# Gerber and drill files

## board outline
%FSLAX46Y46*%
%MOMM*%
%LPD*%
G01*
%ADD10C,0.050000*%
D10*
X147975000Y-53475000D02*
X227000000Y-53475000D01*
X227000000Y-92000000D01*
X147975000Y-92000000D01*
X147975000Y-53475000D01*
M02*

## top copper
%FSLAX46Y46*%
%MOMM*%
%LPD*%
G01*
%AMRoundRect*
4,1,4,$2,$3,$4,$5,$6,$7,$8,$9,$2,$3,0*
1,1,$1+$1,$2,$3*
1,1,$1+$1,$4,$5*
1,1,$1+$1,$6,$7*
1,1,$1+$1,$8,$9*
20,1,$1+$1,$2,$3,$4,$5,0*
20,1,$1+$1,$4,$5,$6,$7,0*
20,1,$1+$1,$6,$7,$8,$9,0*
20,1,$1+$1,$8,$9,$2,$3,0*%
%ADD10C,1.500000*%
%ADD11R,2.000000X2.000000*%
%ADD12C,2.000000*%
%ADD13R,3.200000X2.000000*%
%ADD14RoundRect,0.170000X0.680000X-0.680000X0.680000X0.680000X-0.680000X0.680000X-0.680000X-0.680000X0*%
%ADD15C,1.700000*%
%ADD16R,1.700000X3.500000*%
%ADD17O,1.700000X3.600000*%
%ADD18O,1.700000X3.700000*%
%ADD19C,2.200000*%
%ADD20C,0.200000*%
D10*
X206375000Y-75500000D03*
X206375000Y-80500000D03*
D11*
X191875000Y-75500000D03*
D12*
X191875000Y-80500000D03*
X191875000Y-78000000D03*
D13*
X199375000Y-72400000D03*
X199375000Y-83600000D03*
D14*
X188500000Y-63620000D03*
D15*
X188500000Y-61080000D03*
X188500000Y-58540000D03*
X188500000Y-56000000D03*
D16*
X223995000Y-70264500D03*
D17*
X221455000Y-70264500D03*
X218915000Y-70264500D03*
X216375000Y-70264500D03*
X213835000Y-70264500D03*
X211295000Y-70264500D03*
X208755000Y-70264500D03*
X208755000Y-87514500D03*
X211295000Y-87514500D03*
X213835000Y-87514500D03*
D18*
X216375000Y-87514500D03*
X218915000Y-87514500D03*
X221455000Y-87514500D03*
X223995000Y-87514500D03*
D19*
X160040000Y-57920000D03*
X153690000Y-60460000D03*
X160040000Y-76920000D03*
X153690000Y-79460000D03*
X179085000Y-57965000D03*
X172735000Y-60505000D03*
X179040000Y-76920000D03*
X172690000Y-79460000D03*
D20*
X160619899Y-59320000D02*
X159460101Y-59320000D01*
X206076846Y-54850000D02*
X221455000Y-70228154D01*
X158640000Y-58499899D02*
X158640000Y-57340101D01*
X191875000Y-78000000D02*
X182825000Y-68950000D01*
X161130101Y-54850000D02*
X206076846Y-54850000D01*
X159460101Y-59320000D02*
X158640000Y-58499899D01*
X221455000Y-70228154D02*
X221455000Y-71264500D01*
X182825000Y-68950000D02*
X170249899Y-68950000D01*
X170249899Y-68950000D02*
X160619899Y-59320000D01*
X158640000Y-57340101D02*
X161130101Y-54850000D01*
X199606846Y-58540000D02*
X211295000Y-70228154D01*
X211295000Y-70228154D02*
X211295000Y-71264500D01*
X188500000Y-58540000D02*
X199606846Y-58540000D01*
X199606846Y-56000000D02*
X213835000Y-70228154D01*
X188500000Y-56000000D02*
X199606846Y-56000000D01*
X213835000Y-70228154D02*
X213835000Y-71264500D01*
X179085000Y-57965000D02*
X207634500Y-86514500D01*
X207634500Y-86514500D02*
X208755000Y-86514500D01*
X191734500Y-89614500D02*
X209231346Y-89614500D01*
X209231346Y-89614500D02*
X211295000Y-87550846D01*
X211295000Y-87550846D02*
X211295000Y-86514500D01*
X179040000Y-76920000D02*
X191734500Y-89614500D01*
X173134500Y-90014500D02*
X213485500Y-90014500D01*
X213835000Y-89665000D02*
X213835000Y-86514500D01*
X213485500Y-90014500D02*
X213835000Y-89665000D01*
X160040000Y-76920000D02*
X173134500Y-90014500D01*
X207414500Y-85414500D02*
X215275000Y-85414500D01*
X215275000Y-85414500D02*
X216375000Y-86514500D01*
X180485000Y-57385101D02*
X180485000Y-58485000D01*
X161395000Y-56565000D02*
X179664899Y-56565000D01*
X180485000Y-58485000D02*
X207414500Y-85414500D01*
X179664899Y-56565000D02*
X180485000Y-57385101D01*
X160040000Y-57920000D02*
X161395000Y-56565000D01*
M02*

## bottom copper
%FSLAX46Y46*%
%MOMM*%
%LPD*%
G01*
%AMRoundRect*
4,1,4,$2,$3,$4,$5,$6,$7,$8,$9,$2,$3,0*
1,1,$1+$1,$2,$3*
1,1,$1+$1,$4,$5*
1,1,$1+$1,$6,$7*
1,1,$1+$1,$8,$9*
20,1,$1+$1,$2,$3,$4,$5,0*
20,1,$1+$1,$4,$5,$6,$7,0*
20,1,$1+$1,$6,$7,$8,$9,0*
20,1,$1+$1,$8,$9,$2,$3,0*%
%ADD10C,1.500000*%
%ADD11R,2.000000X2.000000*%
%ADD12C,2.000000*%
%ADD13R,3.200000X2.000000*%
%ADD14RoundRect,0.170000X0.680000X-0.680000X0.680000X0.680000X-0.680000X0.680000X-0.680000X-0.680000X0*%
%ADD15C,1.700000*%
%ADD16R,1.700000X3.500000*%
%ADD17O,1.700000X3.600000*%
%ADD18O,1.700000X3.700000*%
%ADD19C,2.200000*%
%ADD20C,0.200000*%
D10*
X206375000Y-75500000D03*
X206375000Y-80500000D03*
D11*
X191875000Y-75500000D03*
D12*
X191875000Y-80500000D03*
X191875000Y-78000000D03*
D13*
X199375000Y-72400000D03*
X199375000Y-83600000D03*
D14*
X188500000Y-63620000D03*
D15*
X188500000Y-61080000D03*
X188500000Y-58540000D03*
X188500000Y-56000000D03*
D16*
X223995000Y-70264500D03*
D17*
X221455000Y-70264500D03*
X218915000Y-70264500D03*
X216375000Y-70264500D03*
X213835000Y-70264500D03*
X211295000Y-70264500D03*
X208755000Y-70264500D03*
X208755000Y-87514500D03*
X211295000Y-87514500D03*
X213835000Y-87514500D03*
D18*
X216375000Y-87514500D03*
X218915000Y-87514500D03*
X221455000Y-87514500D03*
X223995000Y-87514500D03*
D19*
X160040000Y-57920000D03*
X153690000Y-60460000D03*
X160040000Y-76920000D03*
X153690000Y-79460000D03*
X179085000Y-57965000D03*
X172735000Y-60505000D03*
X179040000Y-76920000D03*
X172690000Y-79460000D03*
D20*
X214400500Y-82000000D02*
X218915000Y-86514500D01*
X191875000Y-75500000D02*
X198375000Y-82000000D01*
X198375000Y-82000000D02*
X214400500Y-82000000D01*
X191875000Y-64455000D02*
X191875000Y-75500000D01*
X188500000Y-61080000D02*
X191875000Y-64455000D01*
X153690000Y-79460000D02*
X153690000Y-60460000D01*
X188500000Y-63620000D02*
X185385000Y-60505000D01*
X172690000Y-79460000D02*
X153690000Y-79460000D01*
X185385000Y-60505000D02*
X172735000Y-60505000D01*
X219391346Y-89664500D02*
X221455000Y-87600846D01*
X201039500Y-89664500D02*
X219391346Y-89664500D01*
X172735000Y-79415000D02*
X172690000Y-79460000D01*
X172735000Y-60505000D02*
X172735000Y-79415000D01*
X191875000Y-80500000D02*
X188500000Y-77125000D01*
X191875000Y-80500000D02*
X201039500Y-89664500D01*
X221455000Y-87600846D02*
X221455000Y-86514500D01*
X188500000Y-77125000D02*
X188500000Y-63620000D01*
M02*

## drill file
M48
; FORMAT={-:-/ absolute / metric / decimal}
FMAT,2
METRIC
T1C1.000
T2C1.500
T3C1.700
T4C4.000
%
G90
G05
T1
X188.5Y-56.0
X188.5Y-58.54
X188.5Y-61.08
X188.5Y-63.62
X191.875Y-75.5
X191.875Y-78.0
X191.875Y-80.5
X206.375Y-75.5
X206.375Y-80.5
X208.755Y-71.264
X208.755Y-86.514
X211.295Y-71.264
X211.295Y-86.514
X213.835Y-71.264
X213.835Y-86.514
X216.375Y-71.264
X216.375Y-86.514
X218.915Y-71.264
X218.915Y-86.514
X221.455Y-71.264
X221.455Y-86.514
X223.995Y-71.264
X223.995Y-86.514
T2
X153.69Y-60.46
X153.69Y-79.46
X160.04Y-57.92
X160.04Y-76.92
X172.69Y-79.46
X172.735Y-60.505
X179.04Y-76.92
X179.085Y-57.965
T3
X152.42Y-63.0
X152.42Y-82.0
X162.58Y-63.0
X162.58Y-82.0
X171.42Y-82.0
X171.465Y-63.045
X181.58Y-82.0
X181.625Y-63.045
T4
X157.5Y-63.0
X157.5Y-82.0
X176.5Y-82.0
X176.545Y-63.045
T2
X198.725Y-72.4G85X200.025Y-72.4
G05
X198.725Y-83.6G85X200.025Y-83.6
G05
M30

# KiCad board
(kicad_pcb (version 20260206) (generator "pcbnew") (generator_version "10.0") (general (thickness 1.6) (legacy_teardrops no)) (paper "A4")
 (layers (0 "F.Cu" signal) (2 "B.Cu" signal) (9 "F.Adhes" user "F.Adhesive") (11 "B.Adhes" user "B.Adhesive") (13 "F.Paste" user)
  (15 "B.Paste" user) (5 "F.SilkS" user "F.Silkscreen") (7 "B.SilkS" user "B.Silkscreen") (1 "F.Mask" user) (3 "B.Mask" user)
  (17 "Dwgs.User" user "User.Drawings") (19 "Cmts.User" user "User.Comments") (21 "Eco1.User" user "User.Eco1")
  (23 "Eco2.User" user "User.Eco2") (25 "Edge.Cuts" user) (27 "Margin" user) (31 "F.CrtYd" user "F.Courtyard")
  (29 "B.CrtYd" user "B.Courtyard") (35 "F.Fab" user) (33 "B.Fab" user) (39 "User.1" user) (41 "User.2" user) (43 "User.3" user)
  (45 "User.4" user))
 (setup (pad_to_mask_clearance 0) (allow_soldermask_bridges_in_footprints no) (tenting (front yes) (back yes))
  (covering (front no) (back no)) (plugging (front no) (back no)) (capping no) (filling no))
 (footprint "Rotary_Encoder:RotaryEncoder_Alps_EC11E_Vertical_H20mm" (layer "F.Cu") (at 191.875 75.5)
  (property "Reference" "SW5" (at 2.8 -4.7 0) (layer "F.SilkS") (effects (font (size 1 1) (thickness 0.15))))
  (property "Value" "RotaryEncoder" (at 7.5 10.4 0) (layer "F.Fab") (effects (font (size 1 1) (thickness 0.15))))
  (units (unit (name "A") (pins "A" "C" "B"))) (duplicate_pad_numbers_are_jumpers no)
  (pad "" thru_hole circle (at 14.5 0) (size 1.5 1.5) (drill 1) (layers "*.Cu" "*.Mask") (remove_unused_layers no))
  (pad "" thru_hole circle (at 14.5 5) (size 1.5 1.5) (drill 1) (layers "*.Cu" "*.Mask") (remove_unused_layers no))
  (pad "A" thru_hole rect (at 0 0) (size 2 2) (drill 1) (layers "*.Cu" "*.Mask") (remove_unused_layers no) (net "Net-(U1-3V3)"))
  (pad "B" thru_hole circle (at 0 5) (size 2 2) (drill 1) (layers "*.Cu" "*.Mask") (remove_unused_layers no) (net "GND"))
  (pad "C" thru_hole circle (at 0 2.5) (size 2 2) (drill 1) (layers "*.Cu" "*.Mask") (remove_unused_layers no) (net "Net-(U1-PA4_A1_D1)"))
  (pad "MP" thru_hole rect (at 7.5 -3.1) (size 3.2 2) (drill oval 2.8 1.5) (layers "*.Cu" "*.Mask") (remove_unused_layers no))
  (pad "MP" thru_hole rect (at 7.5 8.1) (size 3.2 2) (drill oval 2.8 1.5) (layers "*.Cu" "*.Mask") (remove_unused_layers no)))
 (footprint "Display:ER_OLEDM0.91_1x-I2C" (layer "F.Cu") (at 188.5 63.62 90)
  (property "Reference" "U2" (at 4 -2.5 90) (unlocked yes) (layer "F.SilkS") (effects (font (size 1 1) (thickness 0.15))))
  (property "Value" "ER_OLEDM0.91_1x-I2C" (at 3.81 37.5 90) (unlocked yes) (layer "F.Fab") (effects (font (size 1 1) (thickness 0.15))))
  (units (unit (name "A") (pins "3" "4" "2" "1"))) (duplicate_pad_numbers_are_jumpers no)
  (pad "1" thru_hole roundrect (at 0 0 90) (size 1.7 1.7) (drill 1) (layers "*.Cu" "*.Mask") (remove_unused_layers no)
   (roundrect_rratio 0.1) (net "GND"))
  (pad "2" thru_hole circle (at 2.54 0 90) (size 1.7 1.7) (drill 1) (layers "*.Cu" "*.Mask") (remove_unused_layers no) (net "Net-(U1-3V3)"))
  (pad "3" thru_hole circle (at 5.08 0 90) (size 1.7 1.7) (drill 1) (layers "*.Cu" "*.Mask") (remove_unused_layers no)
   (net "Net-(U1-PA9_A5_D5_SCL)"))
  (pad "4" thru_hole circle (at 7.62 0 90) (size 1.7 1.7) (drill 1) (layers "*.Cu" "*.Mask") (remove_unused_layers no)
   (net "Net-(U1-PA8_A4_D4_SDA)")))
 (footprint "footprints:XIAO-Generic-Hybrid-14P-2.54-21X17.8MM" (layer "F.Cu") (at 216.375 78.8895 -90)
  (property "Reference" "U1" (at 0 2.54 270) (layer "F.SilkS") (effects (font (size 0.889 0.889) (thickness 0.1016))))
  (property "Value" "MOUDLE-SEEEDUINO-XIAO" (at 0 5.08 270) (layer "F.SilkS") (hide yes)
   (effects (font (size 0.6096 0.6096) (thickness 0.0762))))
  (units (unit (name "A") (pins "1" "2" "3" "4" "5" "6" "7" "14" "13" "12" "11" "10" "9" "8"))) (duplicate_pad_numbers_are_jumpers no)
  (pad "1" thru_hole rect (at -7.625 -7.62 270) (size 3.5 1.7) (drill 1 (offset -1 0)) (layers "*.Cu" "*.Mask") (remove_unused_layers no)
   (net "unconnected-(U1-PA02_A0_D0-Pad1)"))
  (pad "2" thru_hole oval (at -7.625 -5.08 270) (size 3.6 1.7) (drill 1 (offset -1 0)) (layers "*.Cu" "*.Mask") (remove_unused_layers no)
   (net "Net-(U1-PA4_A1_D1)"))
  (pad "3" thru_hole oval (at -7.625 -2.54 270) (size 3.6 1.7) (drill 1 (offset -1 0)) (layers "*.Cu" "*.Mask") (remove_unused_layers no)
   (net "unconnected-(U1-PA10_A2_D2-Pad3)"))
  (pad "4" thru_hole oval (at -7.625 0 270) (size 3.6 1.7) (drill 1 (offset -1 0)) (layers "*.Cu" "*.Mask") (remove_unused_layers no)
   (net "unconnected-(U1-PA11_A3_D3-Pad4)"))
  (pad "5" thru_hole oval (at -7.625 2.54 270) (size 3.6 1.7) (drill 1 (offset -1 0)) (layers "*.Cu" "*.Mask") (remove_unused_layers no)
   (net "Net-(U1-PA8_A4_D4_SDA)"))
  (pad "6" thru_hole oval (at -7.625 5.08 90) (size 3.6 1.7) (drill 1 (offset 1 0)) (layers "*.Cu" "*.Mask") (remove_unused_layers no)
   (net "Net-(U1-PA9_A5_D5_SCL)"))
  (pad "7" thru_hole oval (at -7.625 7.62 270) (size 3.6 1.7) (drill 1 (offset -1 0)) (layers "*.Cu" "*.Mask") (remove_unused_layers no)
   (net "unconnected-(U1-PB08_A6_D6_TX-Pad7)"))
  (pad "8" thru_hole oval (at 7.625 7.62 270) (size 3.6 1.7) (drill 1 (offset 1 0)) (layers "*.Cu" "*.Mask") (remove_unused_layers no)
   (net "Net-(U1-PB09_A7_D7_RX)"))
  (pad "9" thru_hole oval (at 7.625 5.08 270) (size 3.6 1.7) (drill 1 (offset 1 0)) (layers "*.Cu" "*.Mask") (remove_unused_layers no)
   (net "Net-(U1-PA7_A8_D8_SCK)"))
  (pad "10" thru_hole oval (at 7.625 2.54 270) (size 3.6 1.7) (drill 1 (offset 1 0)) (layers "*.Cu" "*.Mask") (remove_unused_layers no)
   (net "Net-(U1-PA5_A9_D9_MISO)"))
  (pad "11" thru_hole oval (at 7.625 0 270) (size 3.7 1.7) (drill 1 (offset 1 0)) (layers "*.Cu" "*.Mask") (remove_unused_layers no)
   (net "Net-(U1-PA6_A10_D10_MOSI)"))
  (pad "12" thru_hole oval (at 7.625 -2.54 270) (size 3.7 1.7) (drill 1 (offset 1 0)) (layers "*.Cu" "*.Mask") (remove_unused_layers no)
   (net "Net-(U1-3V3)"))
  (pad "13" thru_hole oval (at 7.625 -5.08 270) (size 3.7 1.7) (drill 1 (offset 1 0)) (layers "*.Cu" "*.Mask") (remove_unused_layers no)
   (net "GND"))
  (pad "14" thru_hole oval (at 7.625 -7.62 270) (size 3.7 1.7) (drill 1 (offset 1 0)) (layers "*.Cu" "*.Mask") (remove_unused_layers no)
   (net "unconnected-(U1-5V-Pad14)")))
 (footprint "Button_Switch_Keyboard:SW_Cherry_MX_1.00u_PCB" (layer "F.Cu") (at 160.04 57.92)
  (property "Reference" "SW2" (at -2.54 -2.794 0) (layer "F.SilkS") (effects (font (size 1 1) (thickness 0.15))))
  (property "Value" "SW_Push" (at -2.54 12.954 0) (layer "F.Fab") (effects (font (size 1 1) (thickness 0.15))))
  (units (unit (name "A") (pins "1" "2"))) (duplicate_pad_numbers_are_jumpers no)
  (pad "" np_thru_hole circle (at -7.62 5.08) (size 1.7 1.7) (drill 1.7) (layers "*.Cu" "*.Mask"))
  (pad "" np_thru_hole circle (at -2.54 5.08) (size 4 4) (drill 4) (layers "*.Cu" "*.Mask"))
  (pad "" np_thru_hole circle (at 2.54 5.08) (size 1.7 1.7) (drill 1.7) (layers "*.Cu" "*.Mask"))
  (pad "1" thru_hole circle (at 0 0) (size 2.2 2.2) (drill 1.5) (layers "*.Cu" "*.Mask") (remove_unused_layers no)
   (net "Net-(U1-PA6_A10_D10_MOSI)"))
  (pad "2" thru_hole circle (at -6.35 2.54) (size 2.2 2.2) (drill 1.5) (layers "*.Cu" "*.Mask") (remove_unused_layers no) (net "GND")))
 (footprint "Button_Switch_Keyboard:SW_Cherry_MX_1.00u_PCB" (layer "F.Cu") (at 160.04 76.92)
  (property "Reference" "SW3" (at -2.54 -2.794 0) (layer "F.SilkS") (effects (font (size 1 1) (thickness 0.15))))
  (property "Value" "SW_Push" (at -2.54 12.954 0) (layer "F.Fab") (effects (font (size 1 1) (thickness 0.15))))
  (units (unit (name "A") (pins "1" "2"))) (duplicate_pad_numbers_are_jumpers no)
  (pad "" np_thru_hole circle (at -7.62 5.08) (size 1.7 1.7) (drill 1.7) (layers "*.Cu" "*.Mask"))
  (pad "" np_thru_hole circle (at -2.54 5.08) (size 4 4) (drill 4) (layers "*.Cu" "*.Mask"))
  (pad "" np_thru_hole circle (at 2.54 5.08) (size 1.7 1.7) (drill 1.7) (layers "*.Cu" "*.Mask"))
  (pad "1" thru_hole circle (at 0 0) (size 2.2 2.2) (drill 1.5) (layers "*.Cu" "*.Mask") (remove_unused_layers no)
   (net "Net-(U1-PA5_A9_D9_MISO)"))
  (pad "2" thru_hole circle (at -6.35 2.54) (size 2.2 2.2) (drill 1.5) (layers "*.Cu" "*.Mask") (remove_unused_layers no) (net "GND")))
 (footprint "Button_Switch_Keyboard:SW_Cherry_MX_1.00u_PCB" (layer "F.Cu") (at 179.085 57.965)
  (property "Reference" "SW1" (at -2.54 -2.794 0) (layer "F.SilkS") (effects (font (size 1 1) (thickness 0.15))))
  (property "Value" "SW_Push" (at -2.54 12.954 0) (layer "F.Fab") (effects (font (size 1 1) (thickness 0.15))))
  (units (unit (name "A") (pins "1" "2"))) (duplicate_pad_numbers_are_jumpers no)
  (pad "" np_thru_hole circle (at -7.62 5.08) (size 1.7 1.7) (drill 1.7) (layers "*.Cu" "*.Mask"))
  (pad "" np_thru_hole circle (at -2.54 5.08) (size 4 4) (drill 4) (layers "*.Cu" "*.Mask"))
  (pad "" np_thru_hole circle (at 2.54 5.08) (size 1.7 1.7) (drill 1.7) (layers "*.Cu" "*.Mask"))
  (pad "1" thru_hole circle (at 0 0) (size 2.2 2.2) (drill 1.5) (layers "*.Cu" "*.Mask") (remove_unused_layers no)
   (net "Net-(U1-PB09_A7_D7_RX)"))
  (pad "2" thru_hole circle (at -6.35 2.54) (size 2.2 2.2) (drill 1.5) (layers "*.Cu" "*.Mask") (remove_unused_layers no) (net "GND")))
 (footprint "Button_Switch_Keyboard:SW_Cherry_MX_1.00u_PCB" (layer "F.Cu") (at 179.04 76.92)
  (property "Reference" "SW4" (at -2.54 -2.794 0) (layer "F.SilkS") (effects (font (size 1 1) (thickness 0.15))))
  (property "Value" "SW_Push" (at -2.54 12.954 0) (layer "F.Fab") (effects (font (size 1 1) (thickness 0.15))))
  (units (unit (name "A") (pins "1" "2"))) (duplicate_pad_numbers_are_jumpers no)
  (pad "" np_thru_hole circle (at -7.62 5.08) (size 1.7 1.7) (drill 1.7) (layers "*.Cu" "*.Mask"))
  (pad "" np_thru_hole circle (at -2.54 5.08) (size 4 4) (drill 4) (layers "*.Cu" "*.Mask"))
  (pad "" np_thru_hole circle (at 2.54 5.08) (size 1.7 1.7) (drill 1.7) (layers "*.Cu" "*.Mask"))
  (pad "1" thru_hole circle (at 0 0) (size 2.2 2.2) (drill 1.5) (layers "*.Cu" "*.Mask") (remove_unused_layers no)
   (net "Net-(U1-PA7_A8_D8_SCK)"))
  (pad "2" thru_hole circle (at -6.35 2.54) (size 2.2 2.2) (drill 1.5) (layers "*.Cu" "*.Mask") (remove_unused_layers no) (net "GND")))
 (gr_rect (start 147.975 53.475) (end 227 92) (stroke (width 0.05) (type default)) (fill no) (layer "Edge.Cuts"))
 (segment (start 214.4005 82) (end 218.915 86.5145) (width 0.2) (layer "B.Cu") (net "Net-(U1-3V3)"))
 (segment (start 191.875 75.5) (end 198.375 82) (width 0.2) (layer "B.Cu") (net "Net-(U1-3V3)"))
 (segment (start 198.375 82) (end 214.4005 82) (width 0.2) (layer "B.Cu") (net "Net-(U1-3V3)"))
 (segment (start 191.875 64.455) (end 191.875 75.5) (width 0.2) (layer "B.Cu") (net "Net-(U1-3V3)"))
 (segment (start 188.5 61.08) (end 191.875 64.455) (width 0.2) (layer "B.Cu") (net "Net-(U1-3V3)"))
 (segment (start 153.69 79.46) (end 153.69 60.46) (width 0.2) (layer "B.Cu") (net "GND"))
 (segment (start 188.5 63.62) (end 185.385 60.505) (width 0.2) (layer "B.Cu") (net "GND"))
 (segment (start 172.69 79.46) (end 153.69 79.46) (width 0.2) (layer "B.Cu") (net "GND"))
 (segment (start 185.385 60.505) (end 172.735 60.505) (width 0.2) (layer "B.Cu") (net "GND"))
 (segment (start 219.391346 89.6645) (end 221.455 87.600846) (width 0.2) (layer "B.Cu") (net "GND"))
 (segment (start 201.0395 89.6645) (end 219.391346 89.6645) (width 0.2) (layer "B.Cu") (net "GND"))
 (segment (start 172.735 79.415) (end 172.69 79.46) (width 0.2) (layer "B.Cu") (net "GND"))
 (segment (start 172.735 60.505) (end 172.735 79.415) (width 0.2) (layer "B.Cu") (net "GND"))
 (segment (start 191.875 80.5) (end 188.5 77.125) (width 0.2) (layer "B.Cu") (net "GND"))
 (segment (start 191.875 80.5) (end 201.0395 89.6645) (width 0.2) (layer "B.Cu") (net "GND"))
 (segment (start 221.455 87.600846) (end 221.455 86.5145) (width 0.2) (layer "B.Cu") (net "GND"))
 (segment (start 188.5 77.125) (end 188.5 63.62) (width 0.2) (layer "B.Cu") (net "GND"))
 (segment (start 160.619899 59.32) (end 159.460101 59.32) (width 0.2) (layer "F.Cu") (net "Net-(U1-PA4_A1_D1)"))
 (segment (start 206.076846 54.85) (end 221.455 70.228154) (width 0.2) (layer "F.Cu") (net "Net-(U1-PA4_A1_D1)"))
 (segment (start 158.64 58.499899) (end 158.64 57.340101) (width 0.2) (layer "F.Cu") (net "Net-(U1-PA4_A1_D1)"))
 (segment (start 191.875 78) (end 182.825 68.95) (width 0.2) (layer "F.Cu") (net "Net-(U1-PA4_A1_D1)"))
 (segment (start 161.130101 54.85) (end 206.076846 54.85) (width 0.2) (layer "F.Cu") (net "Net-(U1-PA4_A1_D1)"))
 (segment (start 159.460101 59.32) (end 158.64 58.499899) (width 0.2) (layer "F.Cu") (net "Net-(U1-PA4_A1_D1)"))
 (segment (start 221.455 70.228154) (end 221.455 71.2645) (width 0.2) (layer "F.Cu") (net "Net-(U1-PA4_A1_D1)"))
 (segment (start 182.825 68.95) (end 170.249899 68.95) (width 0.2) (layer "F.Cu") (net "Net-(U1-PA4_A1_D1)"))
 (segment (start 170.249899 68.95) (end 160.619899 59.32) (width 0.2) (layer "F.Cu") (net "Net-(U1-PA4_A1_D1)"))
 (segment (start 158.64 57.340101) (end 161.130101 54.85) (width 0.2) (layer "F.Cu") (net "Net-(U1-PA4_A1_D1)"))
 (segment (start 199.606846 58.54) (end 211.295 70.228154) (width 0.2) (layer "F.Cu") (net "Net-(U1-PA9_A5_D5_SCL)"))
 (segment (start 211.295 70.228154) (end 211.295 71.2645) (width 0.2) (layer "F.Cu") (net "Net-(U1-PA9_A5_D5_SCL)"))
 (segment (start 188.5 58.54) (end 199.606846 58.54) (width 0.2) (layer "F.Cu") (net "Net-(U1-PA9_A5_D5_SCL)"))
 (segment (start 199.606846 56) (end 213.835 70.228154) (width 0.2) (layer "F.Cu") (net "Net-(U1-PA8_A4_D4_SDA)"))
 (segment (start 188.5 56) (end 199.606846 56) (width 0.2) (layer "F.Cu") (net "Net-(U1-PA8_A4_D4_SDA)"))
 (segment (start 213.835 70.228154) (end 213.835 71.2645) (width 0.2) (layer "F.Cu") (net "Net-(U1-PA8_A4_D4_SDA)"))
 (segment (start 179.085 57.965) (end 207.6345 86.5145) (width 0.2) (layer "F.Cu") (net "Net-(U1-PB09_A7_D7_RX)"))
 (segment (start 207.6345 86.5145) (end 208.755 86.5145) (width 0.2) (layer "F.Cu") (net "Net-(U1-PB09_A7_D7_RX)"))
 (segment (start 191.7345 89.6145) (end 209.231346 89.6145) (width 0.2) (layer "F.Cu") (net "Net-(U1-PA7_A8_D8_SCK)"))
 (segment (start 209.231346 89.6145) (end 211.295 87.550846) (width 0.2) (layer "F.Cu") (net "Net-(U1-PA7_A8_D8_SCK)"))
 (segment (start 211.295 87.550846) (end 211.295 86.5145) (width 0.2) (layer "F.Cu") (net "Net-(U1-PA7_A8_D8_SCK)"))
 (segment (start 179.04 76.92) (end 191.7345 89.6145) (width 0.2) (layer "F.Cu") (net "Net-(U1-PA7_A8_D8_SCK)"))
 (segment (start 173.1345 90.0145) (end 213.4855 90.0145) (width 0.2) (layer "F.Cu") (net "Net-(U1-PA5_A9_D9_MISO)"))
 (segment (start 213.835 89.665) (end 213.835 86.5145) (width 0.2) (layer "F.Cu") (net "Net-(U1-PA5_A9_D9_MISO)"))
 (segment (start 213.4855 90.0145) (end 213.835 89.665) (width 0.2) (layer "F.Cu") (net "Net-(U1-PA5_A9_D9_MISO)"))
 (segment (start 160.04 76.92) (end 173.1345 90.0145) (width 0.2) (layer "F.Cu") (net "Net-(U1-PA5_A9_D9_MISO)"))
 (segment (start 207.4145 85.4145) (end 215.275 85.4145) (width 0.2) (layer "F.Cu") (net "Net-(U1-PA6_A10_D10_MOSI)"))
 (segment (start 215.275 85.4145) (end 216.375 86.5145) (width 0.2) (layer "F.Cu") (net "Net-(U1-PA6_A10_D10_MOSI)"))
 (segment (start 180.485 57.385101) (end 180.485 58.485) (width 0.2) (layer "F.Cu") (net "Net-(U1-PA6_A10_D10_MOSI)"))
 (segment (start 161.395 56.565) (end 179.664899 56.565) (width 0.2) (layer "F.Cu") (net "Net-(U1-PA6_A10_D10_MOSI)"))
 (segment (start 180.485 58.485) (end 207.4145 85.4145) (width 0.2) (layer "F.Cu") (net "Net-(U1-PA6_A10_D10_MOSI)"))
 (segment (start 179.664899 56.565) (end 180.485 57.385101) (width 0.2) (layer "F.Cu") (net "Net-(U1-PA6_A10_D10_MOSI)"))
 (segment (start 160.04 57.92) (end 161.395 56.565) (width 0.2) (layer "F.Cu") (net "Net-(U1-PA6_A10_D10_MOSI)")))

